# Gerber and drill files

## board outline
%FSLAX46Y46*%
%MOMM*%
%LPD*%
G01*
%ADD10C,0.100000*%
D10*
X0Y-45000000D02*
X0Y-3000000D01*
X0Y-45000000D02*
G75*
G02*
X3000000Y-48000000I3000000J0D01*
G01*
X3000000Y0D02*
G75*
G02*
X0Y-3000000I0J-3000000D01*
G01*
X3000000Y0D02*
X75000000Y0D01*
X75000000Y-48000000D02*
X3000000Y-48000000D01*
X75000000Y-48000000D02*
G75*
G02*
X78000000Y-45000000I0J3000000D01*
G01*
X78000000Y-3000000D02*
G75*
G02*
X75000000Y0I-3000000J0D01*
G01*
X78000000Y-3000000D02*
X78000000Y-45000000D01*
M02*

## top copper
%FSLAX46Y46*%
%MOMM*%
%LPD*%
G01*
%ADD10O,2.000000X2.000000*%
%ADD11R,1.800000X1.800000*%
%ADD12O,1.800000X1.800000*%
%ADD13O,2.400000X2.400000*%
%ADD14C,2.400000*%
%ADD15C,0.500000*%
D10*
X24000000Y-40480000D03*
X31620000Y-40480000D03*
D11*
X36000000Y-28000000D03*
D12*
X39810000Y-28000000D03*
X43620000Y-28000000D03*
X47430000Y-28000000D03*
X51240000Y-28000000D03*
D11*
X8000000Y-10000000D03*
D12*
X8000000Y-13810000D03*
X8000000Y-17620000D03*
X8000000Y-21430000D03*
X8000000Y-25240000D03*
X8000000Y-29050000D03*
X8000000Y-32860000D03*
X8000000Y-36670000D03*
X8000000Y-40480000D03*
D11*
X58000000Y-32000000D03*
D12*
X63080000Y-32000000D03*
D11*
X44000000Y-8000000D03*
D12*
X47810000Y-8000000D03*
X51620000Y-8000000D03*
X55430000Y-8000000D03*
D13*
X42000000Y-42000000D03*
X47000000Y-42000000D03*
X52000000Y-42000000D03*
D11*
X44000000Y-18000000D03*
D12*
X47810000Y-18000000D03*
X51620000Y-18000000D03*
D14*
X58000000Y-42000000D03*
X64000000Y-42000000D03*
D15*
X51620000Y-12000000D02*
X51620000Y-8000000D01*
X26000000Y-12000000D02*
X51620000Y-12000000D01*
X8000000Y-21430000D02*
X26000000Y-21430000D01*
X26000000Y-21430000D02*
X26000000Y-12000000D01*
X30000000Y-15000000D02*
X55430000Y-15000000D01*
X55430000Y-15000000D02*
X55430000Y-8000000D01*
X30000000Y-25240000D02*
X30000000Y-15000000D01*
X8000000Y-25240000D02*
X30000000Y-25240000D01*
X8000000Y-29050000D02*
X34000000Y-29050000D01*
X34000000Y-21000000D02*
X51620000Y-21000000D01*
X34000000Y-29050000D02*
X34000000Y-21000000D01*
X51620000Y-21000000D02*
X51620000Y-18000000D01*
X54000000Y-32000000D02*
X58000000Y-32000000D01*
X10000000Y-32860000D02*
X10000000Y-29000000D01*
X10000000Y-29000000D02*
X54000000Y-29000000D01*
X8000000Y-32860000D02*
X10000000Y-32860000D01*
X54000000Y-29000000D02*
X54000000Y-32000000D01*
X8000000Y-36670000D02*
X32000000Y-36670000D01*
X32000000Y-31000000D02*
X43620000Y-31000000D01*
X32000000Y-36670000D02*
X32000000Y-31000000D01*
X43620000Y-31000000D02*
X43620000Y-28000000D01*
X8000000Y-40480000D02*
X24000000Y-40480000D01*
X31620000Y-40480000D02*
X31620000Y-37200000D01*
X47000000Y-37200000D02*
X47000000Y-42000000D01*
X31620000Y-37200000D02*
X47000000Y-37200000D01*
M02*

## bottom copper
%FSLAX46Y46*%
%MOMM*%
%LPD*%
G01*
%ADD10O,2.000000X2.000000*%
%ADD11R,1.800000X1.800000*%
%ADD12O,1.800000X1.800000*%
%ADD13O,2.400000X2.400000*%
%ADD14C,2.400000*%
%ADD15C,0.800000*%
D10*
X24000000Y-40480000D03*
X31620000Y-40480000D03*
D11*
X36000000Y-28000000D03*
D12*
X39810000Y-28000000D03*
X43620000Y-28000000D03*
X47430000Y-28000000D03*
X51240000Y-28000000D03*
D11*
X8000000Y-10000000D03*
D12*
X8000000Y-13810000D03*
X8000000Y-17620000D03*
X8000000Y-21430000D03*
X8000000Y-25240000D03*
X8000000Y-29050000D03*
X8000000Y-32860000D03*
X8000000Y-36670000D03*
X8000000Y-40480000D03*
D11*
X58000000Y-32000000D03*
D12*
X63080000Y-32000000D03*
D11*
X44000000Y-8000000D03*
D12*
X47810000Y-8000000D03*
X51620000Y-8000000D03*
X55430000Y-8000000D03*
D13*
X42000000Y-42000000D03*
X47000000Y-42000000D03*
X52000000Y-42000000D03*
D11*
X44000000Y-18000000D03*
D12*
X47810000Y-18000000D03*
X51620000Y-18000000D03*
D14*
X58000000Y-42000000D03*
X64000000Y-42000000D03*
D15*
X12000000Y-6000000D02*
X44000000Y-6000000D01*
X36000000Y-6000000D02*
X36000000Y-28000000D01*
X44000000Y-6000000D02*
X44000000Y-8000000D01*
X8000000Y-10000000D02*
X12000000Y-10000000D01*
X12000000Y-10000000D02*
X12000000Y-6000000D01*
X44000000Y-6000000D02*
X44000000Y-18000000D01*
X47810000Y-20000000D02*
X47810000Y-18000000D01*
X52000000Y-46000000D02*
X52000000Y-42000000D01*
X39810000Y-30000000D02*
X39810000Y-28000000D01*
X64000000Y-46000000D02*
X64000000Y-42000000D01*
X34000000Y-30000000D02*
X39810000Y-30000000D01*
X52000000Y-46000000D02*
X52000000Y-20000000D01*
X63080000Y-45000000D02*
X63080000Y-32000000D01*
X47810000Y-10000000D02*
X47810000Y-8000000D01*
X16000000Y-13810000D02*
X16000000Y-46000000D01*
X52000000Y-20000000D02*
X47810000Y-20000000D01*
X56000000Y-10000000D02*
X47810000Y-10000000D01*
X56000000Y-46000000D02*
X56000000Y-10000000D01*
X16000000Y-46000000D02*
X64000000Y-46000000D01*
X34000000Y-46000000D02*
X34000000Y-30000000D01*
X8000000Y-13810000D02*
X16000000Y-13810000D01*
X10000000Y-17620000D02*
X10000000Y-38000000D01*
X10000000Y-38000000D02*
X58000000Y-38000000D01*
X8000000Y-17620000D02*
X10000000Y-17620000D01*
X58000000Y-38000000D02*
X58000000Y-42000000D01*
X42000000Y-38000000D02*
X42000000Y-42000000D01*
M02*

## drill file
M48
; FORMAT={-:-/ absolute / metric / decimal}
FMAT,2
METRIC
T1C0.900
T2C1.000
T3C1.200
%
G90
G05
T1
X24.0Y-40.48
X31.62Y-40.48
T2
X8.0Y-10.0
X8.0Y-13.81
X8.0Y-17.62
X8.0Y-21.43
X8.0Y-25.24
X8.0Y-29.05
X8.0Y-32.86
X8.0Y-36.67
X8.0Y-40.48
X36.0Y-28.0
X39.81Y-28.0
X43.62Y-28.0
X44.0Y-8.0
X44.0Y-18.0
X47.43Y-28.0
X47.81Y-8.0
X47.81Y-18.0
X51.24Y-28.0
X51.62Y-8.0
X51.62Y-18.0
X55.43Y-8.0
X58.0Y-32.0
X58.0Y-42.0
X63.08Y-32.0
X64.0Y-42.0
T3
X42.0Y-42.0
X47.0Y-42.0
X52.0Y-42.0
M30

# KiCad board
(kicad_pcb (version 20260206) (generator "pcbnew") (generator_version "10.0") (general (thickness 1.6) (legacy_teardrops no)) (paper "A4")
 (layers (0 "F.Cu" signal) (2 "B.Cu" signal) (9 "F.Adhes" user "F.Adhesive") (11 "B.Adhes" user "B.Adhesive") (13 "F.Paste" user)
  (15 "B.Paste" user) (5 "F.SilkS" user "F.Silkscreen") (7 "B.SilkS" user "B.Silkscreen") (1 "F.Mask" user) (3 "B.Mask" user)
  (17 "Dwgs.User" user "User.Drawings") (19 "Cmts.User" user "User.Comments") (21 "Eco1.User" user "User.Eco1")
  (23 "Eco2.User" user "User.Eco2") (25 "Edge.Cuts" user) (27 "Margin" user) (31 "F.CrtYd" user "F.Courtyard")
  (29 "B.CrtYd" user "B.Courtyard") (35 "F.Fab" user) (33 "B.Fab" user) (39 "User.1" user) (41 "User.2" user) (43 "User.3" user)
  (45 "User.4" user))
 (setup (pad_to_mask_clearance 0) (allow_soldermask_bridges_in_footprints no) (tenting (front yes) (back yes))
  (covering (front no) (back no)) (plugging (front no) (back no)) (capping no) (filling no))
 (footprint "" (layer "F.Cu") (at 27.81 40.48)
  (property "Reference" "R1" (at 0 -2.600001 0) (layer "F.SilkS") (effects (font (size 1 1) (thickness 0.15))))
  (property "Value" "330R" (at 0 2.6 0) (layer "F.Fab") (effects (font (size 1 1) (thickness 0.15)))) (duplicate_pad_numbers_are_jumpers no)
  (pad "1" thru_hole oval (at -3.81 0) (size 2 2) (drill 0.9) (layers "*.Cu" "*.Mask") (remove_unused_layers no) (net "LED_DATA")
   (thermal_bridge_angle 45))
  (pad "2" thru_hole oval (at 3.81 0) (size 2 2) (drill 0.9) (layers "*.Cu" "*.Mask") (remove_unused_layers no) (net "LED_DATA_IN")
   (thermal_bridge_angle 45)))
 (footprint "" (layer "F.Cu") (at 36 28)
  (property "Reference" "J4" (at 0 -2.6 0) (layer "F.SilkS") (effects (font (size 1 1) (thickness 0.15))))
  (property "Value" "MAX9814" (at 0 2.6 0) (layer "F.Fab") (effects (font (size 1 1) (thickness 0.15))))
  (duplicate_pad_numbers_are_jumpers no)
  (pad "1" thru_hole rect (at 0 0) (size 1.8 1.8) (drill 1) (layers "*.Cu" "*.Mask") (remove_unused_layers no) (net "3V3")
   (thermal_bridge_angle 45))
  (pad "2" thru_hole oval (at 3.81 0) (size 1.8 1.8) (drill 1) (layers "*.Cu" "*.Mask") (remove_unused_layers no) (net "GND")
   (thermal_bridge_angle 45))
  (pad "3" thru_hole oval (at 7.62 0) (size 1.8 1.8) (drill 1) (layers "*.Cu" "*.Mask") (remove_unused_layers no) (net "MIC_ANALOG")
   (thermal_bridge_angle 45))
  (pad "4" thru_hole oval (at 11.43 0) (size 1.8 1.8) (drill 1) (layers "*.Cu" "*.Mask") (remove_unused_layers no) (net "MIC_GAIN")
   (thermal_bridge_angle 45))
  (pad "5" thru_hole oval (at 15.24 0) (size 1.8 1.8) (drill 1) (layers "*.Cu" "*.Mask") (remove_unused_layers no) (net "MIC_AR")
   (thermal_bridge_angle 45)))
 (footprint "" (layer "F.Cu") (at 8 10)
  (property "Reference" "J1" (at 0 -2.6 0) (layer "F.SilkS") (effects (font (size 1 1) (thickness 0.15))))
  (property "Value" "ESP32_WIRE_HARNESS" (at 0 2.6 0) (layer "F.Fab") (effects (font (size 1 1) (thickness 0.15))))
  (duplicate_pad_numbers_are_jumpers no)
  (pad "1" thru_hole rect (at 0 0) (size 1.8 1.8) (drill 1) (layers "*.Cu" "*.Mask") (remove_unused_layers no) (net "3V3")
   (thermal_bridge_angle 45))
  (pad "2" thru_hole oval (at 0 3.81) (size 1.8 1.8) (drill 1) (layers "*.Cu" "*.Mask") (remove_unused_layers no) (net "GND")
   (thermal_bridge_angle 45))
  (pad "3" thru_hole oval (at 0 7.62) (size 1.8 1.8) (drill 1) (layers "*.Cu" "*.Mask") (remove_unused_layers no) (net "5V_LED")
   (thermal_bridge_angle 45))
  (pad "4" thru_hole oval (at 0 11.43) (size 1.8 1.8) (drill 1) (layers "*.Cu" "*.Mask") (remove_unused_layers no) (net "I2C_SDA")
   (thermal_bridge_angle 45))
  (pad "5" thru_hole oval (at 0 15.24) (size 1.8 1.8) (drill 1) (layers "*.Cu" "*.Mask") (remove_unused_layers no) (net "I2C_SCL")
   (thermal_bridge_angle 45))
  (pad "6" thru_hole oval (at 0 19.05) (size 1.8 1.8) (drill 1) (layers "*.Cu" "*.Mask") (remove_unused_layers no) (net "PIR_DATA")
   (thermal_bridge_angle 45))
  (pad "7" thru_hole oval (at 0 22.86) (size 1.8 1.8) (drill 1) (layers "*.Cu" "*.Mask") (remove_unused_layers no) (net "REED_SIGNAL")
   (thermal_bridge_angle 45))
  (pad "8" thru_hole oval (at 0 26.67) (size 1.8 1.8) (drill 1) (layers "*.Cu" "*.Mask") (remove_unused_layers no) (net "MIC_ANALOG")
   (thermal_bridge_angle 45))
  (pad "9" thru_hole oval (at 0 30.48) (size 1.8 1.8) (drill 1) (layers "*.Cu" "*.Mask") (remove_unused_layers no) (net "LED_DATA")
   (thermal_bridge_angle 45)))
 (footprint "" (layer "F.Cu") (at 58 32)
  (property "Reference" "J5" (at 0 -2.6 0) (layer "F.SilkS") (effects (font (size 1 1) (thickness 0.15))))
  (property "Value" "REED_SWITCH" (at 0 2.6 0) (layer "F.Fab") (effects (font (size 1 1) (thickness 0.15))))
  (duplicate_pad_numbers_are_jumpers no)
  (pad "1" thru_hole rect (at 0 0) (size 1.8 1.8) (drill 1) (layers "*.Cu" "*.Mask") (remove_unused_layers no) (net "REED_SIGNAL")
   (thermal_bridge_angle 45))
  (pad "2" thru_hole oval (at 5.08 0) (size 1.8 1.8) (drill 1) (layers "*.Cu" "*.Mask") (remove_unused_layers no) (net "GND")
   (thermal_bridge_angle 45)))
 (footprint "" (layer "F.Cu") (at 44 8)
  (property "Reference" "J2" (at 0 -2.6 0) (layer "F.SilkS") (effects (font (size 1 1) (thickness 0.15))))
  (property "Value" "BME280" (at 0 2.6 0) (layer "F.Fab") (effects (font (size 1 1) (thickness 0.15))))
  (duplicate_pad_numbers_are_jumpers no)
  (pad "1" thru_hole rect (at 0 0) (size 1.8 1.8) (drill 1) (layers "*.Cu" "*.Mask") (remove_unused_layers no) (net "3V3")
   (thermal_bridge_angle 45))
  (pad "2" thru_hole oval (at 3.81 0) (size 1.8 1.8) (drill 1) (layers "*.Cu" "*.Mask") (remove_unused_layers no) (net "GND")
   (thermal_bridge_angle 45))
  (pad "3" thru_hole oval (at 7.62 0) (size 1.8 1.8) (drill 1) (layers "*.Cu" "*.Mask") (remove_unused_layers no) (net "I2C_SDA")
   (thermal_bridge_angle 45))
  (pad "4" thru_hole oval (at 11.43 0) (size 1.8 1.8) (drill 1) (layers "*.Cu" "*.Mask") (remove_unused_layers no) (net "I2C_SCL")
   (thermal_bridge_angle 45)))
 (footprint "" (layer "F.Cu") (at 42 42)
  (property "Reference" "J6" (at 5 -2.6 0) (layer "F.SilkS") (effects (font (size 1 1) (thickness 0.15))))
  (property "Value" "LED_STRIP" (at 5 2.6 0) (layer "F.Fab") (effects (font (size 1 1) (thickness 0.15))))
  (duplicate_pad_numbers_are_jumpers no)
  (pad "1" thru_hole oval (at 0 0) (size 2.4 2.4) (drill 1.2) (layers "*.Cu" "*.Mask") (remove_unused_layers no) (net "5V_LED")
   (thermal_bridge_angle 45))
  (pad "2" thru_hole oval (at 5 0) (size 2.4 2.4) (drill 1.2) (layers "*.Cu" "*.Mask") (remove_unused_layers no) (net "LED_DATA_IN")
   (thermal_bridge_angle 45))
  (pad "3" thru_hole oval (at 10 0) (size 2.4 2.4) (drill 1.2) (layers "*.Cu" "*.Mask") (remove_unused_layers no) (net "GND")
   (thermal_bridge_angle 45)))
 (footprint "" (layer "F.Cu") (at 44 18)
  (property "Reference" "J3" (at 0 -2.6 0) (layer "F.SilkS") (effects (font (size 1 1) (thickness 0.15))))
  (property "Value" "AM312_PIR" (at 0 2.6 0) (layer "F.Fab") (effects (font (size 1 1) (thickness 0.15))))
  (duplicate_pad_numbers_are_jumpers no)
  (pad "1" thru_hole rect (at 0 0) (size 1.8 1.8) (drill 1) (layers "*.Cu" "*.Mask") (remove_unused_layers no) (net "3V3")
   (thermal_bridge_angle 45))
  (pad "2" thru_hole oval (at 3.81 0) (size 1.8 1.8) (drill 1) (layers "*.Cu" "*.Mask") (remove_unused_layers no) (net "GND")
   (thermal_bridge_angle 45))
  (pad "3" thru_hole oval (at 7.62 0) (size 1.8 1.8) (drill 1) (layers "*.Cu" "*.Mask") (remove_unused_layers no) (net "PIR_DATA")
   (thermal_bridge_angle 45)))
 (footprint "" (layer "F.Cu") (at 61 42)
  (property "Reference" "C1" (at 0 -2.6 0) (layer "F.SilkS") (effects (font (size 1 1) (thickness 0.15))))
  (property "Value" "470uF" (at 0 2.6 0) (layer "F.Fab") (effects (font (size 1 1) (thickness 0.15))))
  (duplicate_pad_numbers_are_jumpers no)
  (pad "1" thru_hole circle (at -3 0) (size 2.4 2.4) (drill 1) (layers "*.Cu" "*.Mask") (remove_unused_layers no) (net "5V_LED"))
  (pad "2" thru_hole circle (at 3 0) (size 2.4 2.4) (drill 1) (layers "*.Cu" "*.Mask") (remove_unused_layers no) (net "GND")))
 (gr_line (start 0 45) (end 0 3) (stroke (width 0.1) (type default)) (layer "Edge.Cuts"))
 (gr_arc (start 0 45) (mid 5.12132 42.87868) (end 3 48) (stroke (width 0.1) (type default)) (layer "Edge.Cuts"))
 (gr_arc (start 3 0) (mid 5.12132 5.12132) (end 0 3) (stroke (width 0.1) (type default)) (layer "Edge.Cuts"))
 (gr_line (start 3 0) (end 75 0) (stroke (width 0.1) (type default)) (layer "Edge.Cuts"))
 (gr_line (start 75 48) (end 3 48) (stroke (width 0.1) (type default)) (layer "Edge.Cuts"))
 (gr_arc (start 75 48) (mid 72.87868 42.87868) (end 78 45) (stroke (width 0.1) (type default)) (layer "Edge.Cuts"))
 (gr_arc (start 78 3) (mid 72.87868 5.12132) (end 75 0) (stroke (width 0.1) (type default)) (layer "Edge.Cuts"))
 (gr_line (start 78 3) (end 78 45) (stroke (width 0.1) (type default)) (layer "Edge.Cuts"))
 (segment (start 12 6) (end 44 6) (width 0.8) (layer "B.Cu") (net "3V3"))
 (segment (start 36 6) (end 36 28) (width 0.8) (layer "B.Cu") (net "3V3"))
 (segment (start 44 6) (end 44 8) (width 0.8) (layer "B.Cu") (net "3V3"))
 (segment (start 8 10) (end 12 10) (width 0.8) (layer "B.Cu") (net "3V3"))
 (segment (start 12 10) (end 12 6) (width 0.8) (layer "B.Cu") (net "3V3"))
 (segment (start 44 6) (end 44 18) (width 0.8) (layer "B.Cu") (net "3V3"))
 (segment (start 47.81 20) (end 47.81 18) (width 0.8) (layer "B.Cu") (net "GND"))
 (segment (start 52 46) (end 52 42) (width 0.8) (layer "B.Cu") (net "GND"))
 (segment (start 39.81 30) (end 39.81 28) (width 0.8) (layer "B.Cu") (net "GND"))
 (segment (start 64 46) (end 64 42) (width 0.8) (layer "B.Cu") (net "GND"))
 (segment (start 34 30) (end 39.81 30) (width 0.8) (layer "B.Cu") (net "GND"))
 (segment (start 52 46) (end 52 20) (width 0.8) (layer "B.Cu") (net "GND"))
 (segment (start 63.08 45) (end 63.08 32) (width 0.8) (layer "B.Cu") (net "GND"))
 (segment (start 47.81 10) (end 47.81 8) (width 0.8) (layer "B.Cu") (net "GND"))
 (segment (start 16 13.81) (end 16 46) (width 0.8) (layer "B.Cu") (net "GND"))
 (segment (start 52 20) (end 47.81 20) (width 0.8) (layer "B.Cu") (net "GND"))
 (segment (start 56 10) (end 47.81 10) (width 0.8) (layer "B.Cu") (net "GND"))
 (segment (start 56 46) (end 56 10) (width 0.8) (layer "B.Cu") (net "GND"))
 (segment (start 16 46) (end 64 46) (width 0.8) (layer "B.Cu") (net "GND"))
 (segment (start 34 46) (end 34 30) (width 0.8) (layer "B.Cu") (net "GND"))
 (segment (start 8 13.81) (end 16 13.81) (width 0.8) (layer "B.Cu") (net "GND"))
 (segment (start 10 17.62) (end 10 38) (width 0.8) (layer "B.Cu") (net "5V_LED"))
 (segment (start 10 38) (end 58 38) (width 0.8) (layer "B.Cu") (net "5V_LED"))
 (segment (start 8 17.62) (end 10 17.62) (width 0.8) (layer "B.Cu") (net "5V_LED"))
 (segment (start 58 38) (end 58 42) (width 0.8) (layer "B.Cu") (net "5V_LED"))
 (segment (start 42 38) (end 42 42) (width 0.8) (layer "B.Cu") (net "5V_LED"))
 (segment (start 51.62 12) (end 51.62 8) (width 0.5) (layer "F.Cu") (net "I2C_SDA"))
 (segment (start 26 12) (end 51.62 12) (width 0.5) (layer "F.Cu") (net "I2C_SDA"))
 (segment (start 8 21.43) (end 26 21.43) (width 0.5) (layer "F.Cu") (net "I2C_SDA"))
 (segment (start 26 21.43) (end 26 12) (width 0.5) (layer "F.Cu") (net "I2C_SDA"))
 (segment (start 30 15) (end 55.43 15) (width 0.5) (layer "F.Cu") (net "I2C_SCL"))
 (segment (start 55.43 15) (end 55.43 8) (width 0.5) (layer "F.Cu") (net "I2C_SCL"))
 (segment (start 30 25.24) (end 30 15) (width 0.5) (layer "F.Cu") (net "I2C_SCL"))
 (segment (start 8 25.24) (end 30 25.24) (width 0.5) (layer "F.Cu") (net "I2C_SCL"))
 (segment (start 8 29.05) (end 34 29.05) (width 0.5) (layer "F.Cu") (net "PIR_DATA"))
 (segment (start 34 21) (end 51.62 21) (width 0.5) (layer "F.Cu") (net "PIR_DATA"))
 (segment (start 34 29.05) (end 34 21) (width 0.5) (layer "F.Cu") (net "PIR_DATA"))
 (segment (start 51.62 21) (end 51.62 18) (width 0.5) (layer "F.Cu") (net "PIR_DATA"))
 (segment (start 54 32) (end 58 32) (width 0.5) (layer "F.Cu") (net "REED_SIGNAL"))
 (segment (start 10 32.86) (end 10 29) (width 0.5) (layer "F.Cu") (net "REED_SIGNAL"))
 (segment (start 10 29) (end 54 29) (width 0.5) (layer "F.Cu") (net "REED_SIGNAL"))
 (segment (start 8 32.86) (end 10 32.86) (width 0.5) (layer "F.Cu") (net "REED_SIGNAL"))
 (segment (start 54 29) (end 54 32) (width 0.5) (layer "F.Cu") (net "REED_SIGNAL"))
 (segment (start 8 36.67) (end 32 36.67) (width 0.5) (layer "F.Cu") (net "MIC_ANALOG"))
 (segment (start 32 31) (end 43.62 31) (width 0.5) (layer "F.Cu") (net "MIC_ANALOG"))
 (segment (start 32 36.67) (end 32 31) (width 0.5) (layer "F.Cu") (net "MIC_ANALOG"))
 (segment (start 43.62 31) (end 43.62 28) (width 0.5) (layer "F.Cu") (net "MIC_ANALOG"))
 (segment (start 8 40.48) (end 24 40.48) (width 0.5) (layer "F.Cu") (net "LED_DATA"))
 (segment (start 31.62 40.48) (end 31.62 37.2) (width 0.5) (layer "F.Cu") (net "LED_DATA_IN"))
 (segment (start 47 37.2) (end 47 42) (width 0.5) (layer "F.Cu") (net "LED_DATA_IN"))
 (segment (start 31.62 37.2) (end 47 37.2) (width 0.5) (layer "F.Cu") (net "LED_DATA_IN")))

